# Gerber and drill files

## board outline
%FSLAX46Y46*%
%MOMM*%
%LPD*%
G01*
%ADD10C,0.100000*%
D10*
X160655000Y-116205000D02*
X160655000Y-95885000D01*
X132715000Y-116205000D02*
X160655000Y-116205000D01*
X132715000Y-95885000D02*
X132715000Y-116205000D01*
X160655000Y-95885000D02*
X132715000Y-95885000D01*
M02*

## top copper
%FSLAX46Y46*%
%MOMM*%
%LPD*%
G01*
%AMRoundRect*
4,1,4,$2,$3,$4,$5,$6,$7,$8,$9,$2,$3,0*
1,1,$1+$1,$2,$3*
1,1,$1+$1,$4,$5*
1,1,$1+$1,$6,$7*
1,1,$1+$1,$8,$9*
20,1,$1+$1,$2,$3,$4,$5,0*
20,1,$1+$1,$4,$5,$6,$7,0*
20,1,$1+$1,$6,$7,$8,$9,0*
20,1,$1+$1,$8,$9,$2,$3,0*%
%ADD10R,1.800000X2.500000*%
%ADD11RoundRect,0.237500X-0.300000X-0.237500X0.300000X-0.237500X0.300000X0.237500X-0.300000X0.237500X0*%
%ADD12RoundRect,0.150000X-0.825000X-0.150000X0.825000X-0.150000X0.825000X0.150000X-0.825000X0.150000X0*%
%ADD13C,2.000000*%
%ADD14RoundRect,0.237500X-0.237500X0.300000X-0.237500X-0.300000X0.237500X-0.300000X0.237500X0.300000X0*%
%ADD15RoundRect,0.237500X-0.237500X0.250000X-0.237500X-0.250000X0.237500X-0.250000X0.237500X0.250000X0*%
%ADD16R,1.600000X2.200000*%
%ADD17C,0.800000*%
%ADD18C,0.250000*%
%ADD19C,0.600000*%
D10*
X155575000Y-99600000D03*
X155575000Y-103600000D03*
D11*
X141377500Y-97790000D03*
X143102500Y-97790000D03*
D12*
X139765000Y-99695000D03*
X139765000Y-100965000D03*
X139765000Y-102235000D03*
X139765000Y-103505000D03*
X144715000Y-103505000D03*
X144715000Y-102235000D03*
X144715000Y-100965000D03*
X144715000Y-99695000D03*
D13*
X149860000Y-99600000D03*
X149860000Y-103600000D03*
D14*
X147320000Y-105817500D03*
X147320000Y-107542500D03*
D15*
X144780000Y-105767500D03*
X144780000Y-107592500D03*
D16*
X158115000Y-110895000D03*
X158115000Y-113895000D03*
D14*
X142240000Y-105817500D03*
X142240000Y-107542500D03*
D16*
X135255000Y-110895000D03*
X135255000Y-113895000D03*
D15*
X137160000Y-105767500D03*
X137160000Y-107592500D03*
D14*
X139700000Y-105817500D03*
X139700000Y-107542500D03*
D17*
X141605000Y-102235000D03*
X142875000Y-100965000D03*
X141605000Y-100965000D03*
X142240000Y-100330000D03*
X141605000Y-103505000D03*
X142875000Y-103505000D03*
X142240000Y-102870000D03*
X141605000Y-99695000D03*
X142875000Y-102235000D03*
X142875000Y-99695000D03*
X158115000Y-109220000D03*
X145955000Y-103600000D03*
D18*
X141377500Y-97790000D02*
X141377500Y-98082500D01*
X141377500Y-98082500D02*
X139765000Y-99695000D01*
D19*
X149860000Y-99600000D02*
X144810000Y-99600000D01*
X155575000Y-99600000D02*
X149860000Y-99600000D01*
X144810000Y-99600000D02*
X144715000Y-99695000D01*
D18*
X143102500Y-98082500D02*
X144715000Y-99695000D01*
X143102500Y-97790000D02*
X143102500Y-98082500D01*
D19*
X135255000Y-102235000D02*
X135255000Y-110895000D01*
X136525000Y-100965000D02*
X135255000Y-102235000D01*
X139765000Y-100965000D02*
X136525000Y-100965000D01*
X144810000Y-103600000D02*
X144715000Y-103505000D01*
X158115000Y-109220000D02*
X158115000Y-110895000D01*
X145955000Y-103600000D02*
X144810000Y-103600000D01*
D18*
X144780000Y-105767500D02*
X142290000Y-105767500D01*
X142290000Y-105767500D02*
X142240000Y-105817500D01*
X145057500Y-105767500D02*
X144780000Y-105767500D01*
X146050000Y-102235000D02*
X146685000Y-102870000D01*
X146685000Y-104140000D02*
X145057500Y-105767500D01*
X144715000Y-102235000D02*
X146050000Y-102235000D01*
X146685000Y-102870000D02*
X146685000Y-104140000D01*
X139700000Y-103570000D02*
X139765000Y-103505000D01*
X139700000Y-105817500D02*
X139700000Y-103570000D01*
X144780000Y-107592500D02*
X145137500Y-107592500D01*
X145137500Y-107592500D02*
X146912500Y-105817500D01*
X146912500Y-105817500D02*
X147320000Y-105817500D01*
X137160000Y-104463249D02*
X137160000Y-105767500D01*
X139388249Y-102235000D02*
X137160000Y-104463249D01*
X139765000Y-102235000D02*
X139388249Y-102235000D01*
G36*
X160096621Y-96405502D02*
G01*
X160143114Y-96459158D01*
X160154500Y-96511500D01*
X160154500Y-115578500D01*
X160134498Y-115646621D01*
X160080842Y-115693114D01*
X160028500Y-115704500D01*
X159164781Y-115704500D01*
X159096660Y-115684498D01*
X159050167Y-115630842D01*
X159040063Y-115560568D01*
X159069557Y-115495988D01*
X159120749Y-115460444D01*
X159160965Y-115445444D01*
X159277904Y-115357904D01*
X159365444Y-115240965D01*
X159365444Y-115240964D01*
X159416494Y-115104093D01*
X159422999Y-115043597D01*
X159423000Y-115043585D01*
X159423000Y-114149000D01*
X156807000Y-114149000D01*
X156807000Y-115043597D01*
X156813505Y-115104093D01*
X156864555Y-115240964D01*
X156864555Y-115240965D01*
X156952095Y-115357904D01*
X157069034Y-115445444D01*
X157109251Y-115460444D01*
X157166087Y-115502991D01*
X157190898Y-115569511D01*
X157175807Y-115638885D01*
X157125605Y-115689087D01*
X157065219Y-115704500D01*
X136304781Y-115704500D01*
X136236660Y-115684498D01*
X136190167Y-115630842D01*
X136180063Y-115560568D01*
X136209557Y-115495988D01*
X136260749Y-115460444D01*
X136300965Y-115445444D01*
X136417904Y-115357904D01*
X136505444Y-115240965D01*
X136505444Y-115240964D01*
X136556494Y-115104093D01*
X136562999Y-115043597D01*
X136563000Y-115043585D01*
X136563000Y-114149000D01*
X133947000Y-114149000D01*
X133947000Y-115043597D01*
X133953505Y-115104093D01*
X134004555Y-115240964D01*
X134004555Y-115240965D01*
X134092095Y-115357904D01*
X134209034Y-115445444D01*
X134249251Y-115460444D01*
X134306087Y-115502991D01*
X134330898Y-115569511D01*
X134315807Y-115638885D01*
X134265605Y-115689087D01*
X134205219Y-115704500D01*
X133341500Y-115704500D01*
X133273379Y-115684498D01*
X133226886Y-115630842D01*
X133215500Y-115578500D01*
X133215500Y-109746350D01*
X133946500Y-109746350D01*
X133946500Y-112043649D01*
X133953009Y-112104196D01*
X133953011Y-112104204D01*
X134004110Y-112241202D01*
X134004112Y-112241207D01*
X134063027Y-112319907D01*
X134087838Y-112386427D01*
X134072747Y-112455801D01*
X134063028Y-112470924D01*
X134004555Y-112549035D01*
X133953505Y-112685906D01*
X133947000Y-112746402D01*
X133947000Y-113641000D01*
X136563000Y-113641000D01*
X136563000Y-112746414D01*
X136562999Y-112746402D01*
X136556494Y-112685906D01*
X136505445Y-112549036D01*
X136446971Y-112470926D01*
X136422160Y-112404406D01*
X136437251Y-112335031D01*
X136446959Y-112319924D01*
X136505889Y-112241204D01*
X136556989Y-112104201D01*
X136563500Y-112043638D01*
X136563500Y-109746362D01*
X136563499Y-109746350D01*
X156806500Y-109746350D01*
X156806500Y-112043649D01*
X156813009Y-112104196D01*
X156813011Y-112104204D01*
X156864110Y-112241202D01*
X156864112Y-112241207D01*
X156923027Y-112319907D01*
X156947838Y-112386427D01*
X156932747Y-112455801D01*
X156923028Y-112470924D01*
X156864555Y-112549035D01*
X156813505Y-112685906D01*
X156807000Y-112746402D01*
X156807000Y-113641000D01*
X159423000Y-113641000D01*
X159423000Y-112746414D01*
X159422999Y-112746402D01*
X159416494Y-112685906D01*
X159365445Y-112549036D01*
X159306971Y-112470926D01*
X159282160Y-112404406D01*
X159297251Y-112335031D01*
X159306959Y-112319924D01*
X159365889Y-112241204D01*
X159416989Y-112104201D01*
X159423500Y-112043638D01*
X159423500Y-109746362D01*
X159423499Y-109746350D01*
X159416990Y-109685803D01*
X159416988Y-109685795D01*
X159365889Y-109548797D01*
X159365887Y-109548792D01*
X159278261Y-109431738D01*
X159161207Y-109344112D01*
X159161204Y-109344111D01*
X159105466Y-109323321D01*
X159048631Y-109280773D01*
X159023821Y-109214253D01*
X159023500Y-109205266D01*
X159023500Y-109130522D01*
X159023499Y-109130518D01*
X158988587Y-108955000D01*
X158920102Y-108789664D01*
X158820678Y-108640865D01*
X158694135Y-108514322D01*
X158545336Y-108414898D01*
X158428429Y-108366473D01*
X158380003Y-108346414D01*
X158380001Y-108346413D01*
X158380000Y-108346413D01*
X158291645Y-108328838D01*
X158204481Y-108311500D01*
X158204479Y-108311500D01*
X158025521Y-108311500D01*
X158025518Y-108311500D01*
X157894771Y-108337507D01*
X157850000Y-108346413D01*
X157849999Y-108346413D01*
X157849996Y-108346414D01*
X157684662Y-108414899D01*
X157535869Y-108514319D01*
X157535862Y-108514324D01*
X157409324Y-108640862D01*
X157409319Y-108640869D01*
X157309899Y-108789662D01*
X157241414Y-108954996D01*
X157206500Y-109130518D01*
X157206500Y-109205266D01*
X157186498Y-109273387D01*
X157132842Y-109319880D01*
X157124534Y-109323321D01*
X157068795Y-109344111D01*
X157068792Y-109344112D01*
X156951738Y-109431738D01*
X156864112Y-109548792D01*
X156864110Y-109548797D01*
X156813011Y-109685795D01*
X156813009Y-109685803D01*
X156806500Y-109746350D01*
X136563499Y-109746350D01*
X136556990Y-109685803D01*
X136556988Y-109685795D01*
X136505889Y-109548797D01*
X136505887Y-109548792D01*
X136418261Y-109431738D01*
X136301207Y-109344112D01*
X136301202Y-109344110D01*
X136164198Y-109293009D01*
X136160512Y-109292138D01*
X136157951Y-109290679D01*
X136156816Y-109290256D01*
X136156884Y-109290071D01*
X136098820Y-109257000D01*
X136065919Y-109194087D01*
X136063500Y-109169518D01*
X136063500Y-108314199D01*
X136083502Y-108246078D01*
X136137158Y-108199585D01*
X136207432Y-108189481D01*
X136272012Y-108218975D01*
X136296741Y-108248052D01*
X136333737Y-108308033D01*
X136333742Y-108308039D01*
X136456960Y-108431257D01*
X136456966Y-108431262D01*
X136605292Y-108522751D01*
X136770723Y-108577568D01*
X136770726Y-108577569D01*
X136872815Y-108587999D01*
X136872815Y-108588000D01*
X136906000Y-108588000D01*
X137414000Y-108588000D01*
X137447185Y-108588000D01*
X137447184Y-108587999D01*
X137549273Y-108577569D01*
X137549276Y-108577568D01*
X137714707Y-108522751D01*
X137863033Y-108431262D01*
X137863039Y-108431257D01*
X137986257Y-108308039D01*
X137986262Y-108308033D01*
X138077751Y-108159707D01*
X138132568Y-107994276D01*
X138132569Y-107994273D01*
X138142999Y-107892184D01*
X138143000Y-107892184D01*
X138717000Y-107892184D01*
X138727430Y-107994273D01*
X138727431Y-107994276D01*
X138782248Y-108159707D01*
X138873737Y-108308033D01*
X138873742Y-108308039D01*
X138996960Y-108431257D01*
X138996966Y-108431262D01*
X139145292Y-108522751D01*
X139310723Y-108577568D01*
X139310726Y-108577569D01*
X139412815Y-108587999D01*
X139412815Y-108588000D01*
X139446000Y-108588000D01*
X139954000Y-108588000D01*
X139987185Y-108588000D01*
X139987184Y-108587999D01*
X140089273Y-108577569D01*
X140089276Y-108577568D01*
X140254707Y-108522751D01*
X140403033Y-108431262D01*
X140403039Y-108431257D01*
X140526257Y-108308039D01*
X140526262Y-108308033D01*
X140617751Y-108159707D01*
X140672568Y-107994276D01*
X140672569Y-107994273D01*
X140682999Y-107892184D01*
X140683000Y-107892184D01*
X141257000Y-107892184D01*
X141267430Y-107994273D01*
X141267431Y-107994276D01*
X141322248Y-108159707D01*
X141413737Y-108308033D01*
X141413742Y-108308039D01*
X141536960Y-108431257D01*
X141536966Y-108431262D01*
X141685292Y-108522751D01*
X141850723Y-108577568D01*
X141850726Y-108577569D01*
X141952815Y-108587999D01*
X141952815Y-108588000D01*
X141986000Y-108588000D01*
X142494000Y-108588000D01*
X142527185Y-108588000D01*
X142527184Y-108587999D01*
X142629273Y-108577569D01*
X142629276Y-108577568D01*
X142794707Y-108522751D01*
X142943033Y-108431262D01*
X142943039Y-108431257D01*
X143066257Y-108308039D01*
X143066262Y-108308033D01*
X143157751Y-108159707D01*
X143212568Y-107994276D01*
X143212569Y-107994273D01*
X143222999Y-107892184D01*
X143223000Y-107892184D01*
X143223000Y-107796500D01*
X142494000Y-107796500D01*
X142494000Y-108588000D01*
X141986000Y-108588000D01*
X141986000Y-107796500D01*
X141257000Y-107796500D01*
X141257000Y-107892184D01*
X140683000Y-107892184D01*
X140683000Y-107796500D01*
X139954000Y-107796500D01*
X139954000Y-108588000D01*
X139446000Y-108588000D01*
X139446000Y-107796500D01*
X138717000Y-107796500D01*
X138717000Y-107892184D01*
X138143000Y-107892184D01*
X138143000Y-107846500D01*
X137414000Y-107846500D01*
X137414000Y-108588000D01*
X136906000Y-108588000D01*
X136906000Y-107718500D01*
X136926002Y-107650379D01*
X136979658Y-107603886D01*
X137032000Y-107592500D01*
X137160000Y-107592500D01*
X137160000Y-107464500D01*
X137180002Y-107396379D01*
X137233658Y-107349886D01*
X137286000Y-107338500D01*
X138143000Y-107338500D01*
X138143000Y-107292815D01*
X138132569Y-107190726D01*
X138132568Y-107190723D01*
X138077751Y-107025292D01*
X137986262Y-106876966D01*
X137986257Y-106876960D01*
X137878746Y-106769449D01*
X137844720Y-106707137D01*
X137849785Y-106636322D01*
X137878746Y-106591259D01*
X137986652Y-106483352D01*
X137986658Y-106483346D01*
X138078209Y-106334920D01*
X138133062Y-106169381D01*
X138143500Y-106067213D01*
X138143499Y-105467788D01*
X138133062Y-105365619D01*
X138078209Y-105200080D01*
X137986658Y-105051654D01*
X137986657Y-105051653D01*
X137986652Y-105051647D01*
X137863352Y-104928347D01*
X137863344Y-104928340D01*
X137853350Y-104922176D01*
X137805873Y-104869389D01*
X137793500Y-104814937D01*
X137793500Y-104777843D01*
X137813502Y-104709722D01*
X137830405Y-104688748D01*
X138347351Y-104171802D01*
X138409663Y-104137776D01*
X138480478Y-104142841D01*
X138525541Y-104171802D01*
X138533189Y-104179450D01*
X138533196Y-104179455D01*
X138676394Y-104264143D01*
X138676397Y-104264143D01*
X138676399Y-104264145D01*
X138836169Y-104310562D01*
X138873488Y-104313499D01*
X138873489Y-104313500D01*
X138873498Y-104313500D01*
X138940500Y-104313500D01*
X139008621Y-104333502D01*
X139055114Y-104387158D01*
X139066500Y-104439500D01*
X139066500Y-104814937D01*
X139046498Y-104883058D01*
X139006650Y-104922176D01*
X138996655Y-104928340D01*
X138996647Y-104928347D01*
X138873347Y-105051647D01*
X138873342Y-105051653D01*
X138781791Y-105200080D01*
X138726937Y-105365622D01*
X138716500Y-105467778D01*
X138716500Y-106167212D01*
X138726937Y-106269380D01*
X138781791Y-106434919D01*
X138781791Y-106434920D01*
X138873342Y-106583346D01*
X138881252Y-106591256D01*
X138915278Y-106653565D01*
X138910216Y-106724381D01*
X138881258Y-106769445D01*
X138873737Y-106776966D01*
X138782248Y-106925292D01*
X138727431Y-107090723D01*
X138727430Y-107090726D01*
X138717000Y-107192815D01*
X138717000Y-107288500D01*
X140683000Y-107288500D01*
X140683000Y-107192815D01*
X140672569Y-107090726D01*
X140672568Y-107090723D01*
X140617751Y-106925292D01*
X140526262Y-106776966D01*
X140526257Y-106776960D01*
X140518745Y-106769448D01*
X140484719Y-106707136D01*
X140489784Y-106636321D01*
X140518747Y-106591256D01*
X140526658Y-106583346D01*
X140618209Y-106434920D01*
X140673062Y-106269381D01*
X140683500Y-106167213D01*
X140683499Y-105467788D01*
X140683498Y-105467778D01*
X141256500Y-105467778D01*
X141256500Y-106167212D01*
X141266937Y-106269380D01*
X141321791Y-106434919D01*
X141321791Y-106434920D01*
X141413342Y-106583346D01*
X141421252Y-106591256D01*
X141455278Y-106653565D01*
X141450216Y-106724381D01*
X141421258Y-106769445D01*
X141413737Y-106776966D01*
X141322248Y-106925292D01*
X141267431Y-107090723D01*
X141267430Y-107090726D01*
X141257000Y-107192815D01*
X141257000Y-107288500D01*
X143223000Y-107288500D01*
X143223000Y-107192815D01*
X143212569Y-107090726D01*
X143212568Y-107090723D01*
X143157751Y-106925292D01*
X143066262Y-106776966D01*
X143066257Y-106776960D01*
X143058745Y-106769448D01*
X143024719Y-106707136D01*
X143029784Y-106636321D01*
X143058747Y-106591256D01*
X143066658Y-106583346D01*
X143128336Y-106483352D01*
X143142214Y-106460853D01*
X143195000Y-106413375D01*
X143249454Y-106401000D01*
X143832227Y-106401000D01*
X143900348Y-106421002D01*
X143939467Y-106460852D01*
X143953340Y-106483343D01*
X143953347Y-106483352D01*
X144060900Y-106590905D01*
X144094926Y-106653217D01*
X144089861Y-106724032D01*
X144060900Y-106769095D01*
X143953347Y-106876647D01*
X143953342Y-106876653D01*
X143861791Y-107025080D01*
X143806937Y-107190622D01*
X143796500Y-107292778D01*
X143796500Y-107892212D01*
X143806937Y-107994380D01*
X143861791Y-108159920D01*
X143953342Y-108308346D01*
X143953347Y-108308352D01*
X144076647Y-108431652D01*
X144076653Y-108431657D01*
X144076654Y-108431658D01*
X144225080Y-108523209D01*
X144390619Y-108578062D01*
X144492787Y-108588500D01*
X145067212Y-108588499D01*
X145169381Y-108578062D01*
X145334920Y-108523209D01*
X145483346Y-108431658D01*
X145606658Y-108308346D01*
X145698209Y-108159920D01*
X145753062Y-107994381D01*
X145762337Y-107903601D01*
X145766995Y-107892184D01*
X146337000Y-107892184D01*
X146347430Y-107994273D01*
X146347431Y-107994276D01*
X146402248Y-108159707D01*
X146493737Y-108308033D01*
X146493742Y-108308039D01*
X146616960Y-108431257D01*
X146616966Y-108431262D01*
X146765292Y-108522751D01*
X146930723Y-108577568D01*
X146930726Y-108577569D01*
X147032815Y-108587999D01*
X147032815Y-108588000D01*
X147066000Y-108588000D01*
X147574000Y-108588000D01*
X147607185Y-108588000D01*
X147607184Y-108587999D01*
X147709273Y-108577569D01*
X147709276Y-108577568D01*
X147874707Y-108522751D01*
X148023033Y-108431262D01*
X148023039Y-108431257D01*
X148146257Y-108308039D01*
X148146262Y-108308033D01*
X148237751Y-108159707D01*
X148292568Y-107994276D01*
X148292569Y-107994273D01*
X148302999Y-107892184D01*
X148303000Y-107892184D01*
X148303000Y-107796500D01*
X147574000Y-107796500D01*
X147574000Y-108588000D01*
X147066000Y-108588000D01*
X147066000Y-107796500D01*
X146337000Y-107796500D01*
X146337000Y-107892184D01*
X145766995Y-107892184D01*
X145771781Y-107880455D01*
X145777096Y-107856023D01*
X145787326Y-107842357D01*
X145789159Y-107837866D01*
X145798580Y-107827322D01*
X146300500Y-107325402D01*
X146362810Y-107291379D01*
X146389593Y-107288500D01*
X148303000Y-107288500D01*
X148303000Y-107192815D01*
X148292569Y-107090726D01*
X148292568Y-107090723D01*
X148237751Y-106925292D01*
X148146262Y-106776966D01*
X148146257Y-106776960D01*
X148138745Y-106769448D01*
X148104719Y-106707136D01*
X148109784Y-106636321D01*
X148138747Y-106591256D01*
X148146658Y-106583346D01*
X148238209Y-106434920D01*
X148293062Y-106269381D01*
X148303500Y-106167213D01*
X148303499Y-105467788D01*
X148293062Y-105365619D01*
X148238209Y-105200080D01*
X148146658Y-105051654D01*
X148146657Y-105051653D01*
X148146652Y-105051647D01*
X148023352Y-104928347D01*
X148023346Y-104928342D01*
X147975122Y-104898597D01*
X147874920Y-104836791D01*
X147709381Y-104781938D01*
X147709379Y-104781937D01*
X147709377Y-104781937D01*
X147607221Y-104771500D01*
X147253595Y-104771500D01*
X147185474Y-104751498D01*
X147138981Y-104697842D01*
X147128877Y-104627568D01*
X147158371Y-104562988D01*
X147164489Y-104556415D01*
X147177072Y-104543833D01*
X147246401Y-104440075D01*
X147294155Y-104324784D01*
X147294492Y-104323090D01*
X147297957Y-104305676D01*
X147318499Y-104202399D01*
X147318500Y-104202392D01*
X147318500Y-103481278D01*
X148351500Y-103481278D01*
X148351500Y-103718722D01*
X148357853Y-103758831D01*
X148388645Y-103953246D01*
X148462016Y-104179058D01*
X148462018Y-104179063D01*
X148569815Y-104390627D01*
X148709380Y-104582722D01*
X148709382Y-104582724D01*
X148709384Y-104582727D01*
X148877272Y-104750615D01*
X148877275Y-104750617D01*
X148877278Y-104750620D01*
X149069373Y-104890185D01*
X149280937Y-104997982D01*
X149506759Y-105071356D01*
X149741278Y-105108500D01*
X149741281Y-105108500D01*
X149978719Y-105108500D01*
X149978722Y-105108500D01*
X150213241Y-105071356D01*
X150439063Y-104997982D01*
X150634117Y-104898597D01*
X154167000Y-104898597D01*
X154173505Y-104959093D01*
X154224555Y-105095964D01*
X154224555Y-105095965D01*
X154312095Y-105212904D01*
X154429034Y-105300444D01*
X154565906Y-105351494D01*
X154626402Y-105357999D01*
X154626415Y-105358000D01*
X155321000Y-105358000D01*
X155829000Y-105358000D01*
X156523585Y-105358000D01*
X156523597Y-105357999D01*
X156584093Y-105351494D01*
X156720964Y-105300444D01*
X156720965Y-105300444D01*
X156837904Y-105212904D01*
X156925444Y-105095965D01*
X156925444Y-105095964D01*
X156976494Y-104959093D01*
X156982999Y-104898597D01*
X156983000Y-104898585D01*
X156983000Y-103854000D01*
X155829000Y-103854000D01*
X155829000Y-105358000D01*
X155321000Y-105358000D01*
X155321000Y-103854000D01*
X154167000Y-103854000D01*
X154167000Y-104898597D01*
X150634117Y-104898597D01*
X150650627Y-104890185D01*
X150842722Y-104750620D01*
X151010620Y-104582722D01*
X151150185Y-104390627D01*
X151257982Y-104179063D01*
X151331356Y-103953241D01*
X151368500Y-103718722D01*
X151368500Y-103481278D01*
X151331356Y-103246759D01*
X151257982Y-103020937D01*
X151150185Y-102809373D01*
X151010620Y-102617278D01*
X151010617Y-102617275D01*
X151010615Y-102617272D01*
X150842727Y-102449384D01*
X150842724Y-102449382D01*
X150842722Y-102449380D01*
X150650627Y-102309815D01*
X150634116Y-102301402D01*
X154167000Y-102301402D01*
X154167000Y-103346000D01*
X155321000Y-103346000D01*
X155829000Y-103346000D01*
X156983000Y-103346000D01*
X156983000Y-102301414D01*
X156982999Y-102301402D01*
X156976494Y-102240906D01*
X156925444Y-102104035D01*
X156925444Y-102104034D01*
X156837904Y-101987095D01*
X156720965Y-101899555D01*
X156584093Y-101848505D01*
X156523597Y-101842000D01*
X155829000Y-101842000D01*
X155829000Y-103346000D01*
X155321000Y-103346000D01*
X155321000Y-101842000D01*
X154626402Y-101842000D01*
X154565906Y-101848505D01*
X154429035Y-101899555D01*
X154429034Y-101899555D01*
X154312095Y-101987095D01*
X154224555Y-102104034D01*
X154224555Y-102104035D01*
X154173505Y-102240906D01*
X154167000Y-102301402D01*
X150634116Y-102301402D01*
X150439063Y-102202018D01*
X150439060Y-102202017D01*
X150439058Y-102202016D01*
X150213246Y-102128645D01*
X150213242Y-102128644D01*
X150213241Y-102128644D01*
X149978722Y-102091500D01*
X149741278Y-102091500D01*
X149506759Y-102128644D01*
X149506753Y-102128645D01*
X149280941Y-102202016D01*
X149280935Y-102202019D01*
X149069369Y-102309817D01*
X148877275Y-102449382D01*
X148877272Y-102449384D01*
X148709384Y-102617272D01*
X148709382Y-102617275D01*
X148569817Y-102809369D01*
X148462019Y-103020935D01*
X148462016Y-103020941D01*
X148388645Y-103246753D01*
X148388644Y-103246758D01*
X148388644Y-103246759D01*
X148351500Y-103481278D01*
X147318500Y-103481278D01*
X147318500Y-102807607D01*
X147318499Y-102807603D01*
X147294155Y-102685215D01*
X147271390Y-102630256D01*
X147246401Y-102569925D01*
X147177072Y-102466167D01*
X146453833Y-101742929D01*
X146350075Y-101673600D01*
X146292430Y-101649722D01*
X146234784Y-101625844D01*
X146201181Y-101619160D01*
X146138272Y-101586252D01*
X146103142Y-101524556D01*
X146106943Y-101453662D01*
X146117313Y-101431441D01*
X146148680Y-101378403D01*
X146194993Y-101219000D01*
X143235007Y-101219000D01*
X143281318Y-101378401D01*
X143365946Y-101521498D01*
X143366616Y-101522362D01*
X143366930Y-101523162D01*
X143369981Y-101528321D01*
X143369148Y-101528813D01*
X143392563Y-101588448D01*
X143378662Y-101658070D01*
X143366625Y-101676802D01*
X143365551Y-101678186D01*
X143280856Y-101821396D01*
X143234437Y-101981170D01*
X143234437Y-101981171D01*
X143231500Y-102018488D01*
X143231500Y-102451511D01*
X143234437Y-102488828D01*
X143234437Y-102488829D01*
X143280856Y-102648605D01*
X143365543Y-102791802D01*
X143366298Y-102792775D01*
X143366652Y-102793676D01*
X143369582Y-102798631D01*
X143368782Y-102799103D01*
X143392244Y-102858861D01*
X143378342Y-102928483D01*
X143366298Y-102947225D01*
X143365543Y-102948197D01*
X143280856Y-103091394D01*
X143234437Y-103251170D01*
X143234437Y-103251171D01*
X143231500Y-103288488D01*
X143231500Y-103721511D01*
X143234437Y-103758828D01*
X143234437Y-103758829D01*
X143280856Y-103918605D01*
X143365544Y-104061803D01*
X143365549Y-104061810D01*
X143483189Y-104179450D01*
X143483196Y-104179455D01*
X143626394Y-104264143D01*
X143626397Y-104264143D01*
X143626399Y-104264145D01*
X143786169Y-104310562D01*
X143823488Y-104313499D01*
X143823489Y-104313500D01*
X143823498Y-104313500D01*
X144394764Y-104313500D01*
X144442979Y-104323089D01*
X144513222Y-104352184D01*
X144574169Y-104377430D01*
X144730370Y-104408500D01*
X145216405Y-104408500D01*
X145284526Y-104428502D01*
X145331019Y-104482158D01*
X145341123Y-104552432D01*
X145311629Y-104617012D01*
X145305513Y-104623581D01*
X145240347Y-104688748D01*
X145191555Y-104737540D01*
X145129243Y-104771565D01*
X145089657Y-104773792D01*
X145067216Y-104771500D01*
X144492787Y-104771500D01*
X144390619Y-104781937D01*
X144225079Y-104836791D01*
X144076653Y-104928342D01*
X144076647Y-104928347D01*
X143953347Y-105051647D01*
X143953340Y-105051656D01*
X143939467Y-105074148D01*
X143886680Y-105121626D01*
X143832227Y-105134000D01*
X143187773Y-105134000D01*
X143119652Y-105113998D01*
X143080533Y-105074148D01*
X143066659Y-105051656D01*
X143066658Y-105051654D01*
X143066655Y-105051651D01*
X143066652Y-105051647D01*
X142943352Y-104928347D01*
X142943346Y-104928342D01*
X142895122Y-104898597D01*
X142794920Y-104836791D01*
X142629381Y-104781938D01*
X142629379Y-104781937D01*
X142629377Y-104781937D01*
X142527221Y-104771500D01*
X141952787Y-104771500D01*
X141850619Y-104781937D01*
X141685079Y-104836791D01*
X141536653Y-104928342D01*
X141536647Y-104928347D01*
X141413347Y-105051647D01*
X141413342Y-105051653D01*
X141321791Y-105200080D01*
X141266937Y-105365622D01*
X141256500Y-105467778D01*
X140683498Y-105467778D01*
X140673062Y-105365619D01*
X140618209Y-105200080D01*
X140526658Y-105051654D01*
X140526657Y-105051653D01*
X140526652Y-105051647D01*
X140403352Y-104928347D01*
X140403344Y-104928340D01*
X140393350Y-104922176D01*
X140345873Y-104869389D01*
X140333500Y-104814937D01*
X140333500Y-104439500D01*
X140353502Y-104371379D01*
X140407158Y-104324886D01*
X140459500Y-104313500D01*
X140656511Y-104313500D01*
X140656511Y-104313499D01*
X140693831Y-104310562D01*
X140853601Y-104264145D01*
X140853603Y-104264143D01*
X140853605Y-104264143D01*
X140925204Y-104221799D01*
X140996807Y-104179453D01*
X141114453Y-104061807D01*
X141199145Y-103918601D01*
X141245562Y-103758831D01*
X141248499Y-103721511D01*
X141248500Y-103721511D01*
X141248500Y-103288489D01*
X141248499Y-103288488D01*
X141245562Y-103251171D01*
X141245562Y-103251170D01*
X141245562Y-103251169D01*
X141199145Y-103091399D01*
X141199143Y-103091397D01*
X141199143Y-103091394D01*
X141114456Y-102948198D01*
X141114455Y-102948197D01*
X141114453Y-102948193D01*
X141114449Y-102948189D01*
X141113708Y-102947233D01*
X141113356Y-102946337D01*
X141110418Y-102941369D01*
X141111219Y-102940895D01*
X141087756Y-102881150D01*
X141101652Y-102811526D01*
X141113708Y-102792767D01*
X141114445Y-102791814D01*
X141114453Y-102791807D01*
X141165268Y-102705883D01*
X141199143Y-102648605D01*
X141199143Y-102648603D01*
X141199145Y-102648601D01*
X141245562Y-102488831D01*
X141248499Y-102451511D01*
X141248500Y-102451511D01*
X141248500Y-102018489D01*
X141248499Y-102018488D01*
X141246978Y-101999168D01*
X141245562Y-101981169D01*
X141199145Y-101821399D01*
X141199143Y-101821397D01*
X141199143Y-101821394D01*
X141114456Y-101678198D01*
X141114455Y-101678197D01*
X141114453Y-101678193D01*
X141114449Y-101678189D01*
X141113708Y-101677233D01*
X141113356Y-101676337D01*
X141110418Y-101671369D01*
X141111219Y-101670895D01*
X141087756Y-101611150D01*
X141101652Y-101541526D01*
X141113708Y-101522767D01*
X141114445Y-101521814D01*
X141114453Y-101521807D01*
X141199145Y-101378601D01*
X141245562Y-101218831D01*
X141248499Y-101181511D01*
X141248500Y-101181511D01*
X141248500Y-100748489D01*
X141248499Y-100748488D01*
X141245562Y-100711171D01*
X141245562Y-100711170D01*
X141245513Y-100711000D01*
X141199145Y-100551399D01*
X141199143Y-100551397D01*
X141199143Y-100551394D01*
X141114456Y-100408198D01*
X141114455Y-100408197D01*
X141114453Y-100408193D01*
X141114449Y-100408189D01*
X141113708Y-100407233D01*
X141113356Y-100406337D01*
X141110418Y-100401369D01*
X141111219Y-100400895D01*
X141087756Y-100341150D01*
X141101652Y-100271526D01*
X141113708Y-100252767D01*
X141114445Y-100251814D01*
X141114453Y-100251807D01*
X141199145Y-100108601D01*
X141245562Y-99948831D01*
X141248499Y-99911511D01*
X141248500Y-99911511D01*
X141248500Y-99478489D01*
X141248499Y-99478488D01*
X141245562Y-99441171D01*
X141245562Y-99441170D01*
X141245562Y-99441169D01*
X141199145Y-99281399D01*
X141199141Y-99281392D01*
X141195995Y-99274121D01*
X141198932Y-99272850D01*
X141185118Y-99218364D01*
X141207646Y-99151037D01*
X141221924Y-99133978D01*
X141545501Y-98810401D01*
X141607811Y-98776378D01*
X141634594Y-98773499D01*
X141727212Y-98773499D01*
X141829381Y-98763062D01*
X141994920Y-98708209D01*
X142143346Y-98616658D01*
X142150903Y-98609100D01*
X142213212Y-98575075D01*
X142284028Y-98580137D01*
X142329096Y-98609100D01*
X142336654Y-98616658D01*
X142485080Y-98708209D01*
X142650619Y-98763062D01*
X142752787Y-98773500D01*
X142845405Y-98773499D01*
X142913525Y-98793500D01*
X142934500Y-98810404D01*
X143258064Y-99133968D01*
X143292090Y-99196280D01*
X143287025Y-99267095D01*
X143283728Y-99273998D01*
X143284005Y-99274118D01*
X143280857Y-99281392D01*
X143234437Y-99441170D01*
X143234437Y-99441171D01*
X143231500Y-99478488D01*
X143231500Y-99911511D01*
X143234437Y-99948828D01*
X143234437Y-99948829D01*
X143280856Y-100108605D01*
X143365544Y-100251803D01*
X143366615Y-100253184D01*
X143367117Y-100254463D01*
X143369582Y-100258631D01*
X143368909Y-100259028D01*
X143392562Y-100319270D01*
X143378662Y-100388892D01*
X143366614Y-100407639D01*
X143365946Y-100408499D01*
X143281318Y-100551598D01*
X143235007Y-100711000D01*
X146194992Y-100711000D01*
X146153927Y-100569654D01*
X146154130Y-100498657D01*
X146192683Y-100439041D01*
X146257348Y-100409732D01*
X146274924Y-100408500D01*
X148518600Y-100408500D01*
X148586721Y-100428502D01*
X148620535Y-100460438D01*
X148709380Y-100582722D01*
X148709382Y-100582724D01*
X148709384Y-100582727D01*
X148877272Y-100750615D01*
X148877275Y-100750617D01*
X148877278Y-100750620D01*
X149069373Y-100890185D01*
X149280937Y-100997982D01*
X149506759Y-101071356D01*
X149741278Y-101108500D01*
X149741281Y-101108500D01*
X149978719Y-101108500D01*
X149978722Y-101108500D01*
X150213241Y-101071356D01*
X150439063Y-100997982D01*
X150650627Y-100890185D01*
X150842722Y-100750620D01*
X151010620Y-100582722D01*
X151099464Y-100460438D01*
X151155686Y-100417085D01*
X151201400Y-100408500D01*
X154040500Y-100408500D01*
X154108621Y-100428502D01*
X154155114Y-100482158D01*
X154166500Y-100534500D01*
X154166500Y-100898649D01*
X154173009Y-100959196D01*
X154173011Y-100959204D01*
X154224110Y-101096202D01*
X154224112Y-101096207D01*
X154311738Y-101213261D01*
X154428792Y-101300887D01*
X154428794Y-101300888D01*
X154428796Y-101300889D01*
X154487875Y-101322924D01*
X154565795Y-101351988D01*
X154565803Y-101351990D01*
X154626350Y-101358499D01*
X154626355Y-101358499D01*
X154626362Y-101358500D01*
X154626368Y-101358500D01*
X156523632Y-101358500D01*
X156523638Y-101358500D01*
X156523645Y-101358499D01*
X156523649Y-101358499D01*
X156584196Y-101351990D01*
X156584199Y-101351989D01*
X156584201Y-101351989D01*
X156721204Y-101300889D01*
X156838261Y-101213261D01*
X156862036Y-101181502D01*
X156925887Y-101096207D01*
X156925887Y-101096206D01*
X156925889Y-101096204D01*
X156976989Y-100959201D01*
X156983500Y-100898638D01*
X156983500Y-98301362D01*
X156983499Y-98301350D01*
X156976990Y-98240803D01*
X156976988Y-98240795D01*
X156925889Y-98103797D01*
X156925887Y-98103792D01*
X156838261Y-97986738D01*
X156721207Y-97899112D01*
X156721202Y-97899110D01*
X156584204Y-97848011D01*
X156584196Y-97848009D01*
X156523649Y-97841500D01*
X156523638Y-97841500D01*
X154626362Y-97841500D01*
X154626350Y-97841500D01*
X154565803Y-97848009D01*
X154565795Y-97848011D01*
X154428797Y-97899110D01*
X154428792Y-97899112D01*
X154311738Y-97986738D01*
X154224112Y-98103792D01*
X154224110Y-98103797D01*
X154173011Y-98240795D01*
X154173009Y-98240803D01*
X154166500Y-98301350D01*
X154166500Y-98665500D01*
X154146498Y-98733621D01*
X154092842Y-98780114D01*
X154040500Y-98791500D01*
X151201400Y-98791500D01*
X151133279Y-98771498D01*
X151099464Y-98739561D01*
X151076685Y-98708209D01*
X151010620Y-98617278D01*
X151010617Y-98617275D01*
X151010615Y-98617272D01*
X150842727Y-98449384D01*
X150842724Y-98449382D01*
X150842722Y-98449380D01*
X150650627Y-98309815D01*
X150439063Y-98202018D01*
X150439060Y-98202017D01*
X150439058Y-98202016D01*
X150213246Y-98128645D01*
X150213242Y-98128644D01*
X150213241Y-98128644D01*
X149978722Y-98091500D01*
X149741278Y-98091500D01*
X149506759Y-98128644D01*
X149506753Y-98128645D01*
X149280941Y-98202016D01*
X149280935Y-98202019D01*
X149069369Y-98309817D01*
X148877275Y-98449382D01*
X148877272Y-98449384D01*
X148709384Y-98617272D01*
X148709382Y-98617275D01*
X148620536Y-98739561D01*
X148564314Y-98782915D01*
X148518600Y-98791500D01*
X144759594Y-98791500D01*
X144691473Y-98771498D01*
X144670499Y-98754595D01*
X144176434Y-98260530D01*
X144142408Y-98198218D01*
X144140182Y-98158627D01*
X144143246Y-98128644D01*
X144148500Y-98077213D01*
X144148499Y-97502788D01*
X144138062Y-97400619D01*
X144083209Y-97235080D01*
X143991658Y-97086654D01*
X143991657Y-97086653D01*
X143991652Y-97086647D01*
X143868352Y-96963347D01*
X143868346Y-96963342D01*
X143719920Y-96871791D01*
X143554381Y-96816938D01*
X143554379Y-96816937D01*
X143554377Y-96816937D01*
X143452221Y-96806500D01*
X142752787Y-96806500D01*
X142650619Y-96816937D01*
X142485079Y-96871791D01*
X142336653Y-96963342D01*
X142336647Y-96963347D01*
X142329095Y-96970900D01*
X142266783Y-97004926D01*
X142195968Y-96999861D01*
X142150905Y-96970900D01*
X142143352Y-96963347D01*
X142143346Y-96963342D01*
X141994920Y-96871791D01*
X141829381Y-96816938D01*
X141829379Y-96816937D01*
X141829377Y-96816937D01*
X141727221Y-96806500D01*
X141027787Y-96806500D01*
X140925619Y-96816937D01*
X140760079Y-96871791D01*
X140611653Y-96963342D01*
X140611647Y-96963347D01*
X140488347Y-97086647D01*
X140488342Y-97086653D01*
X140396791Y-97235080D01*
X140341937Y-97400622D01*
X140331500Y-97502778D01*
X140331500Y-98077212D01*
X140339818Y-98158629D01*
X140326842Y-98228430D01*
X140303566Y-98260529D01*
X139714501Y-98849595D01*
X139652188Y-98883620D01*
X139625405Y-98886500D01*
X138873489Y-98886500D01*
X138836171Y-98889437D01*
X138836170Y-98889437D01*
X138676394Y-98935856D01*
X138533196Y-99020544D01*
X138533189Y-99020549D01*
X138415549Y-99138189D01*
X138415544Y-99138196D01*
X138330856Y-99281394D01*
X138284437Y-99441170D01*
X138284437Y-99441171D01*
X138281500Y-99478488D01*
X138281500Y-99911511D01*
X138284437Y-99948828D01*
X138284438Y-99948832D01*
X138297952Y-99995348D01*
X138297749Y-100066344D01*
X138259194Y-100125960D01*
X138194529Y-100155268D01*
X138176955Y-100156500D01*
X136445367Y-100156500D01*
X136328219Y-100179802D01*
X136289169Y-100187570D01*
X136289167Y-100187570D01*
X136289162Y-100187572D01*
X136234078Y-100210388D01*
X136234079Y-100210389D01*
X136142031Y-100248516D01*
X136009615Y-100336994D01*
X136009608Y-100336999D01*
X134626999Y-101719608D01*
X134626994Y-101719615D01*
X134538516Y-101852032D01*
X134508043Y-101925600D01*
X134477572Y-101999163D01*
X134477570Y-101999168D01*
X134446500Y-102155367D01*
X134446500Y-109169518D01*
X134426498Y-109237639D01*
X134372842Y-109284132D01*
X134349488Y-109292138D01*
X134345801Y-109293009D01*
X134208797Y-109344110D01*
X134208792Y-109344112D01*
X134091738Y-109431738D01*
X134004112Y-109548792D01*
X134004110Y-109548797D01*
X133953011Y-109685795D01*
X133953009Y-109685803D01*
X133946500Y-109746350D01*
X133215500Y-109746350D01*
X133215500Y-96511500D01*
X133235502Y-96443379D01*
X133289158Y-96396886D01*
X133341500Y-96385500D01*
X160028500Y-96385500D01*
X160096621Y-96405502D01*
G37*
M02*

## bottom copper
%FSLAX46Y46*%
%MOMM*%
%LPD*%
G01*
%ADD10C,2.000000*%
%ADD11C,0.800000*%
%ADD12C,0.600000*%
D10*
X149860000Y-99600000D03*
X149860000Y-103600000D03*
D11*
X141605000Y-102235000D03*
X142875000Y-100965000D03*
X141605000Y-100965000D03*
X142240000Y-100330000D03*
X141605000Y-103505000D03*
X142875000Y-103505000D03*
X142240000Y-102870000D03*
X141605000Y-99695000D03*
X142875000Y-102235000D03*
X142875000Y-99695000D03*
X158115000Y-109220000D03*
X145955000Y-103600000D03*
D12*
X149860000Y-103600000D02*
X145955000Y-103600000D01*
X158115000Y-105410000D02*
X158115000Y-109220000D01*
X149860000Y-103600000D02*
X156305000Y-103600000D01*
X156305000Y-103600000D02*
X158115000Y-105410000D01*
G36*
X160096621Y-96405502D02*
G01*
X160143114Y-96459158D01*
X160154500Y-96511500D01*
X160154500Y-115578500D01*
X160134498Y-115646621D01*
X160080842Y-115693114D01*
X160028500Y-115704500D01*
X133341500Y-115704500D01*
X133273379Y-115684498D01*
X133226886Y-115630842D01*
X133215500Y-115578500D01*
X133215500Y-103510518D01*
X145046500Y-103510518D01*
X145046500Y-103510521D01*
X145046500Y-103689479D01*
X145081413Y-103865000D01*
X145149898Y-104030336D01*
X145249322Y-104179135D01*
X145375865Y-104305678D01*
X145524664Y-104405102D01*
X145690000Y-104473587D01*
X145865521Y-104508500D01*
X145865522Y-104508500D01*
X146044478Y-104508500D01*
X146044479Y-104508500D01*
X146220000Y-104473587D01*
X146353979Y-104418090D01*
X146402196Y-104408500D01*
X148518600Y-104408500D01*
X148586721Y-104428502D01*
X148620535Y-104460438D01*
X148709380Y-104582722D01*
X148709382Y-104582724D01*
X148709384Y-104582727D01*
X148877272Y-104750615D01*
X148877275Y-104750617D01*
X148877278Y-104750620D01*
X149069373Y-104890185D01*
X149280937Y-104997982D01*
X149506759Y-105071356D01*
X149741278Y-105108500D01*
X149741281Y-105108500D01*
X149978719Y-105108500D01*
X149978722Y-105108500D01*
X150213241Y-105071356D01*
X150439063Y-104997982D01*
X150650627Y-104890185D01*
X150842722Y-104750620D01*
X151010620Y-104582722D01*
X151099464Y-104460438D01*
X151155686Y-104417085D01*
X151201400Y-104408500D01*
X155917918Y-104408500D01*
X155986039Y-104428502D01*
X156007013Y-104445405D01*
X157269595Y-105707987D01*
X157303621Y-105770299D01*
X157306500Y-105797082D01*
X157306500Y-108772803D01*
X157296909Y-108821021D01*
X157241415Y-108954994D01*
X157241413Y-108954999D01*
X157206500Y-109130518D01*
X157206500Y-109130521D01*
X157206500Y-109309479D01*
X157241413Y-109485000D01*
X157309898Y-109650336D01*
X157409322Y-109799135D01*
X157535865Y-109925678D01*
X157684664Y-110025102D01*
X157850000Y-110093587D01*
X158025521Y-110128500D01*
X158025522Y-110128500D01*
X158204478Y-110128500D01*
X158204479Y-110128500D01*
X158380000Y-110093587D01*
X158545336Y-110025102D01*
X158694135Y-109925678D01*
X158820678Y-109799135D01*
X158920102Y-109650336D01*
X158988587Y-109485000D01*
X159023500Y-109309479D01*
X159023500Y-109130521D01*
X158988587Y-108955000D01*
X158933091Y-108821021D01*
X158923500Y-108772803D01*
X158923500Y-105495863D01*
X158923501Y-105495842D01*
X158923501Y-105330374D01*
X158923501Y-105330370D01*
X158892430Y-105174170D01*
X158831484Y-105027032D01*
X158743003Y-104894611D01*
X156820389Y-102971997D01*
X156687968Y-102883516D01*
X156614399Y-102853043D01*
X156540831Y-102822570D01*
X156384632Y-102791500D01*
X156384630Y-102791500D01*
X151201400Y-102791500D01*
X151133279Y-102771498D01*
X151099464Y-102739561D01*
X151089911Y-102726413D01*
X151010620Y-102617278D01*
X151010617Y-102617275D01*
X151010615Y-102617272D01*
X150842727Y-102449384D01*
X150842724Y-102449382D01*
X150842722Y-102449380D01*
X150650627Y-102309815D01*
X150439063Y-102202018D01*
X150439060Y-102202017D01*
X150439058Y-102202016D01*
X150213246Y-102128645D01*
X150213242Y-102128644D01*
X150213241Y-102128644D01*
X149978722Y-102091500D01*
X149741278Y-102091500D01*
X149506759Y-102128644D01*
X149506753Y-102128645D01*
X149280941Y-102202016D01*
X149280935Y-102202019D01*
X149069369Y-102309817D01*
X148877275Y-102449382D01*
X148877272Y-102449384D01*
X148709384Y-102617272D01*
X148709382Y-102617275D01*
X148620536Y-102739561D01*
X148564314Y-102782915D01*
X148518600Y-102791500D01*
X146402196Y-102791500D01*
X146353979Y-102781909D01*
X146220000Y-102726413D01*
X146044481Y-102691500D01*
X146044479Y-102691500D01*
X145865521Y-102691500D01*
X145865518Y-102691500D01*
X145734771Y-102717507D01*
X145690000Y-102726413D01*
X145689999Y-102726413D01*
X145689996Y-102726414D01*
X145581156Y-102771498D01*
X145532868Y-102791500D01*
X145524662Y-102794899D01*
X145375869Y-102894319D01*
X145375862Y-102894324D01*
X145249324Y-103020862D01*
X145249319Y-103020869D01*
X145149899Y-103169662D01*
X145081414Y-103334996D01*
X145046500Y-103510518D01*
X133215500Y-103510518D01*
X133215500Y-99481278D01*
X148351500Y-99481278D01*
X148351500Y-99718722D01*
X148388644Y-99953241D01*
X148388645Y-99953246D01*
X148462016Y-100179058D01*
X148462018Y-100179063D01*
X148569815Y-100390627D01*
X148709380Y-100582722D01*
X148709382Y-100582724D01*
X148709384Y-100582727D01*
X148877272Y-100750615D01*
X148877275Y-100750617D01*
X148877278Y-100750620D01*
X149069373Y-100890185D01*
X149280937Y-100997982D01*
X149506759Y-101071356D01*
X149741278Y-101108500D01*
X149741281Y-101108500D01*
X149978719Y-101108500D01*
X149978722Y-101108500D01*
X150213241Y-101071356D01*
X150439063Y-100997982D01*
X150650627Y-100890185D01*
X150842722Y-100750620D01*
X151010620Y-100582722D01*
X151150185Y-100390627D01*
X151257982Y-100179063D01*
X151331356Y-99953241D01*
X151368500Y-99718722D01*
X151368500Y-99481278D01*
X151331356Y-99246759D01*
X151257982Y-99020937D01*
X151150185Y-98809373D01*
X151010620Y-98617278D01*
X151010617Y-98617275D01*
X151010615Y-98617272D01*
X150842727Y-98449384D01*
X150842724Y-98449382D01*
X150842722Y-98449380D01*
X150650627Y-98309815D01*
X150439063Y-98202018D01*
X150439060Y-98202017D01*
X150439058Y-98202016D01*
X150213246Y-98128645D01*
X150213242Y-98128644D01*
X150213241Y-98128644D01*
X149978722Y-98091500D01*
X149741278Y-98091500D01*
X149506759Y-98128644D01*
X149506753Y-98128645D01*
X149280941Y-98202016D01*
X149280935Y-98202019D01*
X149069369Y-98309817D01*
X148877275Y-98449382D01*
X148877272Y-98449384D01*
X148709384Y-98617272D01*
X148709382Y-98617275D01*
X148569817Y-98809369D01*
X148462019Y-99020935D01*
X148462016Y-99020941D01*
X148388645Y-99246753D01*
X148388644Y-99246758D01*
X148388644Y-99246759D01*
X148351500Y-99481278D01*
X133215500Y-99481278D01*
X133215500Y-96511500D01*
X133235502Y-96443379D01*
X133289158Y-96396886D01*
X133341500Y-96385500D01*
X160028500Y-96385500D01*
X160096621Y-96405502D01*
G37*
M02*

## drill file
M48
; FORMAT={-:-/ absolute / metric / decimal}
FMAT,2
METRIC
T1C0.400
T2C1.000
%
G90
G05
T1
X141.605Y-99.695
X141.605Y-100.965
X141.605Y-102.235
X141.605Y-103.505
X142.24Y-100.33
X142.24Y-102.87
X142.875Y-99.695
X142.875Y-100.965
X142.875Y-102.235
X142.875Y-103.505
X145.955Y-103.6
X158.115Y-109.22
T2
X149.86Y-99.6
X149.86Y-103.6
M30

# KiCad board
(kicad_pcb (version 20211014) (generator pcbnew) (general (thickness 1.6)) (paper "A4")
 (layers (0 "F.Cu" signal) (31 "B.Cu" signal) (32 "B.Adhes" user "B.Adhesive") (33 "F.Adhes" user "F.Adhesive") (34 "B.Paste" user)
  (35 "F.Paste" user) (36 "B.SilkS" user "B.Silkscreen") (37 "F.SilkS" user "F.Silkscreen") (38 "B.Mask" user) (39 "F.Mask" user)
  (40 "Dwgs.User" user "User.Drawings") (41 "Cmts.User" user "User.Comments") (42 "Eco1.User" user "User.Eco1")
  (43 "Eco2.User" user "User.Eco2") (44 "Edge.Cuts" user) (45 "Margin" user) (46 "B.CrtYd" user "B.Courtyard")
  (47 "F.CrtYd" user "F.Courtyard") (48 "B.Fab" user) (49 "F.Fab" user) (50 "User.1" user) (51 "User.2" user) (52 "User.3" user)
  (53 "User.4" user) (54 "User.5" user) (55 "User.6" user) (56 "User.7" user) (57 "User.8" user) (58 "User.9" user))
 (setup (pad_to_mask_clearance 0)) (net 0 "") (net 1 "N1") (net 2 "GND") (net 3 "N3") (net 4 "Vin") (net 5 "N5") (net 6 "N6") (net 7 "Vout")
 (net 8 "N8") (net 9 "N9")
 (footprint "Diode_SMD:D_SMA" (layer "F.Cu") (at 155.575 101.6 -90)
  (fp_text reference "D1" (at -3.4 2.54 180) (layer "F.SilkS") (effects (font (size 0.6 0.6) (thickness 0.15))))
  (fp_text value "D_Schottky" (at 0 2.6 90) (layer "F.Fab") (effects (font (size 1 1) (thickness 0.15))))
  (pad "1" smd rect (at -2 0 270) (size 2.5 1.8) (layers "F.Cu" "F.Paste" "F.Mask") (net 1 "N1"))
  (pad "2" smd rect (at 2 0 270) (size 2.5 1.8) (layers "F.Cu" "F.Paste" "F.Mask") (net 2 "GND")))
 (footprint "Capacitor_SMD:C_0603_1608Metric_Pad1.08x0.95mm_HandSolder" (layer "F.Cu") (at 142.24 97.79)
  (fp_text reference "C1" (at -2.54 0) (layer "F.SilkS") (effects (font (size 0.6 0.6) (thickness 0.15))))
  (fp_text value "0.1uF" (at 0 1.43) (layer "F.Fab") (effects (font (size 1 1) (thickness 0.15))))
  (pad "1" smd roundrect (at -0.8625 0) (size 1.075 0.95) (layers "F.Cu" "F.Paste" "F.Mask") (roundrect_rratio 0.25) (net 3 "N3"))
  (pad "2" smd roundrect (at 0.8625 0) (size 1.075 0.95) (layers "F.Cu" "F.Paste" "F.Mask") (roundrect_rratio 0.25) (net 1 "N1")))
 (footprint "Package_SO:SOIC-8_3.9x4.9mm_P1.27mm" (layer "F.Cu") (at 142.24 101.6)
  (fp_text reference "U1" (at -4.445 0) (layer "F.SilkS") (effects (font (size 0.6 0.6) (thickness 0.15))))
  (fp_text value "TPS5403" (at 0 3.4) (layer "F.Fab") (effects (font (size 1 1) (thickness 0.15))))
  (pad "1" smd roundrect (at -2.475 -1.905) (size 1.95 0.6) (layers "F.Cu" "F.Paste" "F.Mask") (roundrect_rratio 0.25) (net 3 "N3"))
  (pad "2" smd roundrect (at -2.475 -0.635) (size 1.95 0.6) (layers "F.Cu" "F.Paste" "F.Mask") (roundrect_rratio 0.25) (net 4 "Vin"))
  (pad "3" smd roundrect (at -2.475 0.635) (size 1.95 0.6) (layers "F.Cu" "F.Paste" "F.Mask") (roundrect_rratio 0.25) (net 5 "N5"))
  (pad "4" smd roundrect (at -2.475 1.905) (size 1.95 0.6) (layers "F.Cu" "F.Paste" "F.Mask") (roundrect_rratio 0.25) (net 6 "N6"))
  (pad "5" smd roundrect (at 2.475 1.905) (size 1.95 0.6) (layers "F.Cu" "F.Paste" "F.Mask") (roundrect_rratio 0.25) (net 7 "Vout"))
  (pad "6" smd roundrect (at 2.475 0.635) (size 1.95 0.6) (layers "F.Cu" "F.Paste" "F.Mask") (roundrect_rratio 0.25) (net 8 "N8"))
  (pad "7" smd roundrect (at 2.475 -0.635) (size 1.95 0.6) (layers "F.Cu" "F.Paste" "F.Mask") (roundrect_rratio 0.25) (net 2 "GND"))
  (pad "8" smd roundrect (at 2.475 -1.905) (size 1.95 0.6) (layers "F.Cu" "F.Paste" "F.Mask") (roundrect_rratio 0.25) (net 1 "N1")))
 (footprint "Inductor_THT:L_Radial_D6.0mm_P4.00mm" (layer "F.Cu") (at 149.86 99.6 -90)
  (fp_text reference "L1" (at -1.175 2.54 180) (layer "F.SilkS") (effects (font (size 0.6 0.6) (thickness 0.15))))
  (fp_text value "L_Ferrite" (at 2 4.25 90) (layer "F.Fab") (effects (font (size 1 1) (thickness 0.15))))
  (pad "1" thru_hole circle (at 0 0 270) (size 2 2) (drill 1) (layers *.Cu *.Mask) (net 1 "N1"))
  (pad "2" thru_hole circle (at 4 0 270) (size 2 2) (drill 1) (layers *.Cu *.Mask) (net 7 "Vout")))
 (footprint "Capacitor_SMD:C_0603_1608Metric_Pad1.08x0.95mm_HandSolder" (layer "F.Cu") (at 147.32 106.68 -90)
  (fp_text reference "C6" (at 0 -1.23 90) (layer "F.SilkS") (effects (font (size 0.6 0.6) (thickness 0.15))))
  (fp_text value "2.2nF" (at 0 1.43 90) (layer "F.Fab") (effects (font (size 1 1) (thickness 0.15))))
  (pad "1" smd roundrect (at -0.8625 0 270) (size 1.075 0.95) (layers "F.Cu" "F.Paste" "F.Mask") (roundrect_rratio 0.25) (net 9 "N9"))
  (pad "2" smd roundrect (at 0.8625 0 270) (size 1.075 0.95) (layers "F.Cu" "F.Paste" "F.Mask") (roundrect_rratio 0.25) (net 2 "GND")))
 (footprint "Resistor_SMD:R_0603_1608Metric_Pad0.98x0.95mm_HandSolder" (layer "F.Cu") (at 144.78 106.68 -90)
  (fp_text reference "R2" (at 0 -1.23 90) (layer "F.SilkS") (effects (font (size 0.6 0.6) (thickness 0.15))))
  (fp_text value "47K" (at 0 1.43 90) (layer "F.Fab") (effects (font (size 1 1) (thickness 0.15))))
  (pad "1" smd roundrect (at -0.9125 0 270) (size 0.975 0.95) (layers "F.Cu" "F.Paste" "F.Mask") (roundrect_rratio 0.25) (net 8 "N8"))
  (pad "2" smd roundrect (at 0.9125 0 270) (size 0.975 0.95) (layers "F.Cu" "F.Paste" "F.Mask") (roundrect_rratio 0.25) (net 9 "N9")))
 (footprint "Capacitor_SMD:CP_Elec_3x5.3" (layer "F.Cu") (at 158.115 112.395 -90)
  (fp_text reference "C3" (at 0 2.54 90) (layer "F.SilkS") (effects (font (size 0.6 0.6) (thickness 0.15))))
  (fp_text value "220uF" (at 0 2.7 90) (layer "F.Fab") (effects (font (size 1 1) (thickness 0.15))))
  (pad "1" smd rect (at -1.5 0 270) (size 2.2 1.6) (layers "F.Cu" "F.Paste" "F.Mask") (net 7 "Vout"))
  (pad "2" smd rect (at 1.5 0 270) (size 2.2 1.6) (layers "F.Cu" "F.Paste" "F.Mask") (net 2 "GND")))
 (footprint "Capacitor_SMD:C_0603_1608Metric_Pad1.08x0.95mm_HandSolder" (layer "F.Cu") (at 142.24 106.68 -90)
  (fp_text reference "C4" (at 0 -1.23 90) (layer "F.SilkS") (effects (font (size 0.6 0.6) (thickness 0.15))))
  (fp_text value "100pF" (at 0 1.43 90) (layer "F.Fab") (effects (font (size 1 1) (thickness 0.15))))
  (pad "1" smd roundrect (at -0.8625 0 270) (size 1.075 0.95) (layers "F.Cu" "F.Paste" "F.Mask") (roundrect_rratio 0.25) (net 8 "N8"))
  (pad "2" smd roundrect (at 0.8625 0 270) (size 1.075 0.95) (layers "F.Cu" "F.Paste" "F.Mask") (roundrect_rratio 0.25) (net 2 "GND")))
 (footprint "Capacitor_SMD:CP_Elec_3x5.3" (layer "F.Cu") (at 135.255 112.395 -90)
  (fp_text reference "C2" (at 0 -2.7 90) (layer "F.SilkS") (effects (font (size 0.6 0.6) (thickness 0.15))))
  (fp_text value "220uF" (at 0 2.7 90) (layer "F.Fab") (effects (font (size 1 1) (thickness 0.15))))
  (pad "1" smd rect (at -1.5 0 270) (size 2.2 1.6) (layers "F.Cu" "F.Paste" "F.Mask") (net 4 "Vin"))
  (pad "2" smd rect (at 1.5 0 270) (size 2.2 1.6) (layers "F.Cu" "F.Paste" "F.Mask") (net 2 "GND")))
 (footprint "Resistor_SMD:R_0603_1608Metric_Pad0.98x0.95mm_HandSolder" (layer "F.Cu") (at 137.16 106.68 -90)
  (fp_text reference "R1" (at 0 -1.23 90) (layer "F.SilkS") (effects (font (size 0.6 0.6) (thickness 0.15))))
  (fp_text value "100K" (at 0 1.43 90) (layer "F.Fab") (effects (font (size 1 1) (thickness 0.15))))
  (pad "1" smd roundrect (at -0.9125 0 270) (size 0.975 0.95) (layers "F.Cu" "F.Paste" "F.Mask") (roundrect_rratio 0.25) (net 5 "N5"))
  (pad "2" smd roundrect (at 0.9125 0 270) (size 0.975 0.95) (layers "F.Cu" "F.Paste" "F.Mask") (roundrect_rratio 0.25) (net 2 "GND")))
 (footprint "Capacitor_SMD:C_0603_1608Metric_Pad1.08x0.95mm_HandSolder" (layer "F.Cu") (at 139.7 106.68 -90)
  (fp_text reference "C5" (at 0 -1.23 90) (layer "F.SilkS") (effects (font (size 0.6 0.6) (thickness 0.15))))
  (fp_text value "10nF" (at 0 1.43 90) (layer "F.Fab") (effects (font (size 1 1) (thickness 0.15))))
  (pad "1" smd roundrect (at -0.8625 0 270) (size 1.075 0.95) (layers "F.Cu" "F.Paste" "F.Mask") (roundrect_rratio 0.25) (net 6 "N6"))
  (pad "2" smd roundrect (at 0.8625 0 270) (size 1.075 0.95) (layers "F.Cu" "F.Paste" "F.Mask") (roundrect_rratio 0.25) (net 2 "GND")))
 (gr_line (start 160.655 116.205) (end 160.655 95.885) (layer "Edge.Cuts") (width 0.1))
 (gr_line (start 132.715 116.205) (end 160.655 116.205) (layer "Edge.Cuts") (width 0.1))
 (gr_line (start 132.715 95.885) (end 132.715 116.205) (layer "Edge.Cuts") (width 0.1))
 (gr_line (start 160.655 95.885) (end 132.715 95.885) (layer "Edge.Cuts") (width 0.1))
 (segment (start 141.3775 97.79) (end 141.3775 98.0825) (width 0.25) (layer "F.Cu") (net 3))
 (segment (start 141.3775 98.0825) (end 139.765 99.695) (width 0.25) (layer "F.Cu") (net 3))
 (segment (start 149.86 99.6) (end 144.81 99.6) (width 0.6) (layer "F.Cu") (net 1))
 (segment (start 155.575 99.6) (end 149.86 99.6) (width 0.6) (layer "F.Cu") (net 1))
 (segment (start 144.81 99.6) (end 144.715 99.695) (width 0.6) (layer "F.Cu") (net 1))
 (segment (start 143.1025 98.0825) (end 144.715 99.695) (width 0.25) (layer "F.Cu") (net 1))
 (segment (start 143.1025 97.79) (end 143.1025 98.0825) (width 0.25) (layer "F.Cu") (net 1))
 (segment (start 135.255 102.235) (end 135.255 110.895) (width 0.6) (layer "F.Cu") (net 4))
 (segment (start 136.525 100.965) (end 135.255 102.235) (width 0.6) (layer "F.Cu") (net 4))
 (segment (start 139.765 100.965) (end 136.525 100.965) (width 0.6) (layer "F.Cu") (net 4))
 (via (at 141.605 102.235) (size 0.8) (drill 0.4) (layers "F.Cu" "B.Cu") (free) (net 2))
 (via (at 142.875 100.965) (size 0.8) (drill 0.4) (layers "F.Cu" "B.Cu") (free) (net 2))
 (via (at 141.605 100.965) (size 0.8) (drill 0.4) (layers "F.Cu" "B.Cu") (free) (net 2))
 (via (at 142.24 100.33) (size 0.8) (drill 0.4) (layers "F.Cu" "B.Cu") (free) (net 2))
 (via (at 141.605 103.505) (size 0.8) (drill 0.4) (layers "F.Cu" "B.Cu") (free) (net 2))
 (via (at 142.875 103.505) (size 0.8) (drill 0.4) (layers "F.Cu" "B.Cu") (free) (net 2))
 (via (at 142.24 102.87) (size 0.8) (drill 0.4) (layers "F.Cu" "B.Cu") (free) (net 2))
 (via (at 141.605 99.695) (size 0.8) (drill 0.4) (layers "F.Cu" "B.Cu") (free) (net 2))
 (via (at 142.875 102.235) (size 0.8) (drill 0.4) (layers "F.Cu" "B.Cu") (free) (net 2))
 (via (at 142.875 99.695) (size 0.8) (drill 0.4) (layers "F.Cu" "B.Cu") (free) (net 2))
 (segment (start 144.81 103.6) (end 144.715 103.505) (width 0.6) (layer "F.Cu") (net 7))
 (segment (start 158.115 109.22) (end 158.115 110.895) (width 0.6) (layer "F.Cu") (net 7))
 (segment (start 145.955 103.6) (end 144.81 103.6) (width 0.6) (layer "F.Cu") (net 7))
 (via (at 158.115 109.22) (size 0.8) (drill 0.4) (layers "F.Cu" "B.Cu") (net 7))
 (via (at 145.955 103.6) (size 0.8) (drill 0.4) (layers "F.Cu" "B.Cu") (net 7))
 (segment (start 149.86 103.6) (end 145.955 103.6) (width 0.6) (layer "B.Cu") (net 7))
 (segment (start 158.115 105.41) (end 158.115 109.22) (width 0.6) (layer "B.Cu") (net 7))
 (segment (start 149.86 103.6) (end 156.305 103.6) (width 0.6) (layer "B.Cu") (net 7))
 (segment (start 156.305 103.6) (end 158.115 105.41) (width 0.6) (layer "B.Cu") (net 7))
 (segment (start 144.78 105.7675) (end 142.29 105.7675) (width 0.25) (layer "F.Cu") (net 8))
 (segment (start 142.29 105.7675) (end 142.24 105.8175) (width 0.25) (layer "F.Cu") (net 8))
 (segment (start 145.0575 105.7675) (end 144.78 105.7675) (width 0.25) (layer "F.Cu") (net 8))
 (segment (start 146.05 102.235) (end 146.685 102.87) (width 0.25) (layer "F.Cu") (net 8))
 (segment (start 146.685 104.14) (end 145.0575 105.7675) (width 0.25) (layer "F.Cu") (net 8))
 (segment (start 144.715 102.235) (end 146.05 102.235) (width 0.25) (layer "F.Cu") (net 8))
 (segment (start 146.685 102.87) (end 146.685 104.14) (width 0.25) (layer "F.Cu") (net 8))
 (segment (start 139.7 103.57) (end 139.765 103.505) (width 0.25) (layer "F.Cu") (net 6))
 (segment (start 139.7 105.8175) (end 139.7 103.57) (width 0.25) (layer "F.Cu") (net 6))
 (segment (start 144.78 107.5925) (end 145.1375 107.5925) (width 0.25) (layer "F.Cu") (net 9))
 (segment (start 145.1375 107.5925) (end 146.9125 105.8175) (width 0.25) (layer "F.Cu") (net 9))
 (segment (start 146.9125 105.8175) (end 147.32 105.8175) (width 0.25) (layer "F.Cu") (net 9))
 (segment (start 137.16 104.463249) (end 137.16 105.7675) (width 0.25) (layer "F.Cu") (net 5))
 (segment (start 139.388249 102.235) (end 137.16 104.463249) (width 0.25) (layer "F.Cu") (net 5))
 (segment (start 139.765 102.235) (end 139.388249 102.235) (width 0.25) (layer "F.Cu") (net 5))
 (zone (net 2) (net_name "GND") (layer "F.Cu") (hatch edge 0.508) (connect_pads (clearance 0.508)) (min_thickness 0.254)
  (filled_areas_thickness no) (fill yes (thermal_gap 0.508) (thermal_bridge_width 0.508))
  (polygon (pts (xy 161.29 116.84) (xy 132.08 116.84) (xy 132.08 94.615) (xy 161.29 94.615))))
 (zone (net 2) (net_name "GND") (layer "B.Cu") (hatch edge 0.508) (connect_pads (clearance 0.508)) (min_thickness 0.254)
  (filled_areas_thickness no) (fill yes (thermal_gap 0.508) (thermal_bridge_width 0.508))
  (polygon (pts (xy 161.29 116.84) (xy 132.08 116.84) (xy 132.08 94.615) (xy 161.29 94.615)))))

